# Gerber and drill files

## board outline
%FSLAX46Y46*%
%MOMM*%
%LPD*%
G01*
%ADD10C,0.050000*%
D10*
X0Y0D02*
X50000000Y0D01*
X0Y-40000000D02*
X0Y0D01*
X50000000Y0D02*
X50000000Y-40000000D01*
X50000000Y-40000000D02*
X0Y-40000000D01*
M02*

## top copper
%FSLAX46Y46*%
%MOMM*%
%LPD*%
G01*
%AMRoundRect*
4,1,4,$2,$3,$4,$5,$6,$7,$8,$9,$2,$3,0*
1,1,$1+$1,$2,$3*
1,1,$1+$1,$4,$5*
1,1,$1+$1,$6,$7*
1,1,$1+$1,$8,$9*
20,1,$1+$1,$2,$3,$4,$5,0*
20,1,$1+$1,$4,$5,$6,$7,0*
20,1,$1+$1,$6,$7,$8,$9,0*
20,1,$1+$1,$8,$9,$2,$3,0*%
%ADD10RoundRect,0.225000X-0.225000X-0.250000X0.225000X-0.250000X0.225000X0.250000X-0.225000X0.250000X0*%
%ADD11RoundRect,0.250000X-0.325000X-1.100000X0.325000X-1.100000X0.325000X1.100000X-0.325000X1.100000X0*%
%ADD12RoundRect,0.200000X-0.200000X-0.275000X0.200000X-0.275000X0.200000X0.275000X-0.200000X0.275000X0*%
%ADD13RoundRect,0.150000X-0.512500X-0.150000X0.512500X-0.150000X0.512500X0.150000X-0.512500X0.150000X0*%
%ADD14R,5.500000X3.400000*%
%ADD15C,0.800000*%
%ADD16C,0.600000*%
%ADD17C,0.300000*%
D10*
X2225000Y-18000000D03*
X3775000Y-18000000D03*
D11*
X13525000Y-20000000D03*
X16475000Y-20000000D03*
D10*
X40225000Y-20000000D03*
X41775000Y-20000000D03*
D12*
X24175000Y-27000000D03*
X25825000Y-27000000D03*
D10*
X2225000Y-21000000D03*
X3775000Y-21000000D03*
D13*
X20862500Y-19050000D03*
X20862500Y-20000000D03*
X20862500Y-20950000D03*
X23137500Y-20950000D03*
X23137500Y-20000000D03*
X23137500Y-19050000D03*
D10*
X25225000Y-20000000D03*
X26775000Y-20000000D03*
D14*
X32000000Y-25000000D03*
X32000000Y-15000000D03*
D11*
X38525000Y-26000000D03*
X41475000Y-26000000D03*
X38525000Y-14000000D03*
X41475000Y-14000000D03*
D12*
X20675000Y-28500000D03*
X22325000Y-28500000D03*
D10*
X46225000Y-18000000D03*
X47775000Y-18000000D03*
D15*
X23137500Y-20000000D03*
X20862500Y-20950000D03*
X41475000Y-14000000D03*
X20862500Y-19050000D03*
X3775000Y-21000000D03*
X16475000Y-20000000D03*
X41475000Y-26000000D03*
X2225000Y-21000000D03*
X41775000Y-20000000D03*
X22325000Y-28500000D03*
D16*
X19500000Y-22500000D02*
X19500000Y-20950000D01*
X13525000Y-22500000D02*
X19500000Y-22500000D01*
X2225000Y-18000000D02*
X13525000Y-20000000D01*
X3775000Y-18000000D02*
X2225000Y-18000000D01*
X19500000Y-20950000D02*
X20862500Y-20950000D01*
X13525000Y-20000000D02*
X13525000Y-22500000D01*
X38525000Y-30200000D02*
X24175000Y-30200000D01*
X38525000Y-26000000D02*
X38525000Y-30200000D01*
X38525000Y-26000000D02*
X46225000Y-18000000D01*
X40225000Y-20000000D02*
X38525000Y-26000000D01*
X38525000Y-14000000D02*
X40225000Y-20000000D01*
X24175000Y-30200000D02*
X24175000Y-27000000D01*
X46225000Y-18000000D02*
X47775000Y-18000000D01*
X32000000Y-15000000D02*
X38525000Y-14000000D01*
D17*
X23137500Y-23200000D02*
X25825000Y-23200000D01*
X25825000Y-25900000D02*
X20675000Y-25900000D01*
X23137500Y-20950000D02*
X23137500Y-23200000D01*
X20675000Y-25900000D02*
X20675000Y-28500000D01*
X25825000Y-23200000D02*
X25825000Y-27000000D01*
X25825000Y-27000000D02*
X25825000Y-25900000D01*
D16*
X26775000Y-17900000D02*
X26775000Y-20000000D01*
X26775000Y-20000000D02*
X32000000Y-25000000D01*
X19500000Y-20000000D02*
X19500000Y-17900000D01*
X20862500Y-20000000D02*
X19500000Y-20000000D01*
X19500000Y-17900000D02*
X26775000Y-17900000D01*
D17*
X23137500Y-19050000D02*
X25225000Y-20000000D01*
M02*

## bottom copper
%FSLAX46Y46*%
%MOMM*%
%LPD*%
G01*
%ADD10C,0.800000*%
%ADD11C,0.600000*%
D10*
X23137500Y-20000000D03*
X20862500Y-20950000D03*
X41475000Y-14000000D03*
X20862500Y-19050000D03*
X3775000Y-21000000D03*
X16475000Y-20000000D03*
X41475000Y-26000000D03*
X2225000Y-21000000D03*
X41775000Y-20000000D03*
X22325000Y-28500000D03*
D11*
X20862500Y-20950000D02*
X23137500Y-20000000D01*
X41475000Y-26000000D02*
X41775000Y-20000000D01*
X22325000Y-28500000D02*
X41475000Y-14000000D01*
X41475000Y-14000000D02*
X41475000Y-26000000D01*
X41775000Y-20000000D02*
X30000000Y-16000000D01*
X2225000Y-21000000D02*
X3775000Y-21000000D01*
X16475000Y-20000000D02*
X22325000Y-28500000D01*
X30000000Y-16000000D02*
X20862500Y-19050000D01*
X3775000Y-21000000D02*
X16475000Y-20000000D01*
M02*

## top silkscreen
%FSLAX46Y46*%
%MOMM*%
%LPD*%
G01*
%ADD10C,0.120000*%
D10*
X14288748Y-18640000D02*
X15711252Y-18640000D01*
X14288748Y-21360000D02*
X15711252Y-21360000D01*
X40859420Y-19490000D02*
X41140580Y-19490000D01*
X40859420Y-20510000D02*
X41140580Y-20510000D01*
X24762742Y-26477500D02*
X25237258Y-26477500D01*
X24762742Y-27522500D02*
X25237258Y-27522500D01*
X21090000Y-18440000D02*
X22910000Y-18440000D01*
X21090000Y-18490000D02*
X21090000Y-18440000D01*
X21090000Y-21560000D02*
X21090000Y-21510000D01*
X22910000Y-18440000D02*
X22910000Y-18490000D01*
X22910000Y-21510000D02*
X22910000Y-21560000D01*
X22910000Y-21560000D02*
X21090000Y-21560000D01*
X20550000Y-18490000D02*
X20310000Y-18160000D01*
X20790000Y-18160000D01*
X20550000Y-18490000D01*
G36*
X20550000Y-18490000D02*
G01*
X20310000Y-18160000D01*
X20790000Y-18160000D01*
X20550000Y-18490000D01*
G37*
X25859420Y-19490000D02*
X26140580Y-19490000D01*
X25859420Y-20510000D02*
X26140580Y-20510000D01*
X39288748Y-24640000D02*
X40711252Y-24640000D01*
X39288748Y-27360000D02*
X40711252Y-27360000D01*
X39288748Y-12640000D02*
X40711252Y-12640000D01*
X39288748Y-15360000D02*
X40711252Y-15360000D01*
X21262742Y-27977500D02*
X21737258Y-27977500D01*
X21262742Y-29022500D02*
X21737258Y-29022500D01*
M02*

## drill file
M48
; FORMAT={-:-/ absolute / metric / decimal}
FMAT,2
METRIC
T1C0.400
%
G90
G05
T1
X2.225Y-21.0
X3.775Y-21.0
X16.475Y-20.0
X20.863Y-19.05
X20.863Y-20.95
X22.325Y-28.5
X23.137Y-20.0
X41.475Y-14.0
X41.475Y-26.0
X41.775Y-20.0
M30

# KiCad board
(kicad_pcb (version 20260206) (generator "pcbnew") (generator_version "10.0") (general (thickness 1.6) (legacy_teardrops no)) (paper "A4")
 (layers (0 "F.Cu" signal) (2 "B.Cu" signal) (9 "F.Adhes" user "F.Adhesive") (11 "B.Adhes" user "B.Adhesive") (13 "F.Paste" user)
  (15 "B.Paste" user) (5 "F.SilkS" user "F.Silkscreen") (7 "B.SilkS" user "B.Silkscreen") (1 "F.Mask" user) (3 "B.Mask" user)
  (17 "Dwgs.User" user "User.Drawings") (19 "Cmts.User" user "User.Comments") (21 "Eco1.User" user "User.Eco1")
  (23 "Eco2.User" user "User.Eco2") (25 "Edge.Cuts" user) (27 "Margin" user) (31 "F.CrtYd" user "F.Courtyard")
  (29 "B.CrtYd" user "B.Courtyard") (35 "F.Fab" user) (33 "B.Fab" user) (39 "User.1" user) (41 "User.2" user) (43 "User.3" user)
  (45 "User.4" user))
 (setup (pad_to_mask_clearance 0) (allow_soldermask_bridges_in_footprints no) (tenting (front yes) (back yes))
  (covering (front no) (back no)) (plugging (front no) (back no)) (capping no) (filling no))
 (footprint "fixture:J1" (layer "F.Cu") (at 3 18)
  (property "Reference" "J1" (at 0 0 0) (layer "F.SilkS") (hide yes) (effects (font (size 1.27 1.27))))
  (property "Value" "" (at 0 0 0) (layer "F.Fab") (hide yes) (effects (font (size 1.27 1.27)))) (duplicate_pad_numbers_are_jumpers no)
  (pad "1" smd roundrect (at -0.775 0) (size 0.9 0.95) (layers "F.Cu" "F.Mask" "F.Paste") (roundrect_rratio 0.25) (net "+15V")
   (thermal_bridge_angle 45))
  (pad "2" smd roundrect (at 0.775 0) (size 0.9 0.95) (layers "F.Cu" "F.Mask" "F.Paste") (roundrect_rratio 0.25) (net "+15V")
   (thermal_bridge_angle 45)))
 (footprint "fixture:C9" (layer "F.Cu") (at 15 20)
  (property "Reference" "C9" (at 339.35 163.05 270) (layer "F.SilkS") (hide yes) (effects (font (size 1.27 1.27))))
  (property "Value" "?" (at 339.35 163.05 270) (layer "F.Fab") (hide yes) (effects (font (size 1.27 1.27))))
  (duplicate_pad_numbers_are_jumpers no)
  (fp_line (start -0.711252 -1.36) (end 0.711252 -1.36) (stroke (width 0.12) (type solid)) (layer "F.SilkS"))
  (fp_line (start -0.711252 1.36) (end 0.711252 1.36) (stroke (width 0.12) (type solid)) (layer "F.SilkS"))
  (pad "1" smd roundrect (at -1.475 0) (size 1.15 2.7) (layers "F.Cu" "F.Mask" "F.Paste") (roundrect_rratio 0.217391) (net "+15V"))
  (pad "2" smd roundrect (at 1.475 0) (size 1.15 2.7) (layers "F.Cu" "F.Mask" "F.Paste") (roundrect_rratio 0.217391) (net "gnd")))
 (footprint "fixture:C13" (layer "F.Cu") (at 41 20)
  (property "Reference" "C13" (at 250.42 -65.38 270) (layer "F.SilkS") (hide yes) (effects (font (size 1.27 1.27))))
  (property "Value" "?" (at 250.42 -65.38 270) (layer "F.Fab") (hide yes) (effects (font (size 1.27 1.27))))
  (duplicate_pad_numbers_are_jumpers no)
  (fp_line (start -0.14058 -0.51) (end 0.14058 -0.51) (stroke (width 0.12) (type solid)) (layer "F.SilkS"))
  (fp_line (start -0.14058 0.51) (end 0.14058 0.51) (stroke (width 0.12) (type solid)) (layer "F.SilkS"))
  (pad "1" smd roundrect (at -0.775 0) (size 0.9 0.95) (layers "F.Cu" "F.Mask" "F.Paste") (roundrect_rratio 0.25) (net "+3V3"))
  (pad "2" smd roundrect (at 0.775 0) (size 0.9 0.95) (layers "F.Cu" "F.Mask" "F.Paste") (roundrect_rratio 0.25) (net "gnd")))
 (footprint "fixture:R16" (layer "F.Cu") (at 25 27)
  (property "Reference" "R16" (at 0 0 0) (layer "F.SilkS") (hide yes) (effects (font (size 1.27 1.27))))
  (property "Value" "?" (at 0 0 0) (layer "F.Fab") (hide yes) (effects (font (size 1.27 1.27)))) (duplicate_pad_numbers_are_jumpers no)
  (fp_line (start -0.237258 -0.5225) (end 0.237258 -0.5225) (stroke (width 0.12) (type solid)) (layer "F.SilkS"))
  (fp_line (start -0.237258 0.5225) (end 0.237258 0.5225) (stroke (width 0.12) (type solid)) (layer "F.SilkS"))
  (pad "1" smd roundrect (at -0.825 0) (size 0.8 0.95) (layers "F.Cu" "F.Mask" "F.Paste") (roundrect_rratio 0.25) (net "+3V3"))
  (pad "2" smd roundrect (at 0.825 0) (size 0.8 0.95) (layers "F.Cu" "F.Mask" "F.Paste") (roundrect_rratio 0.25) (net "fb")))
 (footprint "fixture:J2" (layer "F.Cu") (at 3 21)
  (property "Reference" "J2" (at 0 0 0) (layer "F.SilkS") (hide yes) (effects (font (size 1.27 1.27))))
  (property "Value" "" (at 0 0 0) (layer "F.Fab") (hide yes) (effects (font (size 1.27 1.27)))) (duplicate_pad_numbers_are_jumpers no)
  (pad "1" smd roundrect (at -0.775 0) (size 0.9 0.95) (layers "F.Cu" "F.Mask" "F.Paste") (roundrect_rratio 0.25) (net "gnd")
   (thermal_bridge_angle 45))
  (pad "2" smd roundrect (at 0.775 0) (size 0.9 0.95) (layers "F.Cu" "F.Mask" "F.Paste") (roundrect_rratio 0.25) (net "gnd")
   (thermal_bridge_angle 45)))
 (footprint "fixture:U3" (layer "F.Cu") (at 22 20)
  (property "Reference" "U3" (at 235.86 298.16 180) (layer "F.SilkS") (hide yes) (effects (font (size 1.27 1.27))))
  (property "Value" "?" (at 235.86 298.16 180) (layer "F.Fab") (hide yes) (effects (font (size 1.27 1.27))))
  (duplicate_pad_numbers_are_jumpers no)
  (fp_line (start -0.91 -1.56) (end 0.91 -1.56) (stroke (width 0.12) (type solid)) (layer "F.SilkS"))
  (fp_line (start -0.91 -1.51) (end -0.91 -1.56) (stroke (width 0.12) (type solid)) (layer "F.SilkS"))
  (fp_line (start -0.91 1.56) (end -0.91 1.51) (stroke (width 0.12) (type solid)) (layer "F.SilkS"))
  (fp_line (start 0.91 -1.56) (end 0.91 -1.51) (stroke (width 0.12) (type solid)) (layer "F.SilkS"))
  (fp_line (start 0.91 1.51) (end 0.91 1.56) (stroke (width 0.12) (type solid)) (layer "F.SilkS"))
  (fp_line (start 0.91 1.56) (end -0.91 1.56) (stroke (width 0.12) (type solid)) (layer "F.SilkS"))
  (fp_poly (pts (xy -1.45 -1.51) (xy -1.69 -1.84) (xy -1.21 -1.84)) (stroke (width 0.12) (type solid)) (fill yes) (layer "F.SilkS"))
  (pad "1" smd roundrect (at -1.1375 -0.95) (size 1.325 0.6) (layers "F.Cu" "F.Mask" "F.Paste") (roundrect_rratio 0.25) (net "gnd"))
  (pad "2" smd roundrect (at -1.1375 0) (size 1.325 0.6) (layers "F.Cu" "F.Mask" "F.Paste") (roundrect_rratio 0.25) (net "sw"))
  (pad "3" smd roundrect (at -1.1375 0.95) (size 1.325 0.6) (layers "F.Cu" "F.Mask" "F.Paste") (roundrect_rratio 0.25) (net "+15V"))
  (pad "4" smd roundrect (at 1.1375 0.95) (size 1.325 0.6) (layers "F.Cu" "F.Mask" "F.Paste") (roundrect_rratio 0.25) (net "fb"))
  (pad "5" smd roundrect (at 1.1375 0) (size 1.325 0.6) (layers "F.Cu" "F.Mask" "F.Paste") (roundrect_rratio 0.25) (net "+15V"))
  (pad "6" smd roundrect (at 1.1375 -0.95) (size 1.325 0.6) (layers "F.Cu" "F.Mask" "F.Paste") (roundrect_rratio 0.25) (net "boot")))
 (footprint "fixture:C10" (layer "F.Cu") (at 26 20)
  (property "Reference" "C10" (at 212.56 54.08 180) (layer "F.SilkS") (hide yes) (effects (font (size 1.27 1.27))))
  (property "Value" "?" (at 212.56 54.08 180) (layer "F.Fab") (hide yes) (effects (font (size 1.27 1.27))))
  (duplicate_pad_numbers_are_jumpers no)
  (fp_line (start -0.14058 -0.51) (end 0.14058 -0.51) (stroke (width 0.12) (type solid)) (layer "F.SilkS"))
  (fp_line (start -0.14058 0.51) (end 0.14058 0.51) (stroke (width 0.12) (type solid)) (layer "F.SilkS"))
  (pad "1" smd roundrect (at -0.775 0) (size 0.9 0.95) (layers "F.Cu" "F.Mask" "F.Paste") (roundrect_rratio 0.25) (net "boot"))
  (pad "2" smd roundrect (at 0.775 0) (size 0.9 0.95) (layers "F.Cu" "F.Mask" "F.Paste") (roundrect_rratio 0.25) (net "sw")))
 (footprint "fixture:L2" (layer "F.Cu") (at 32 20 90)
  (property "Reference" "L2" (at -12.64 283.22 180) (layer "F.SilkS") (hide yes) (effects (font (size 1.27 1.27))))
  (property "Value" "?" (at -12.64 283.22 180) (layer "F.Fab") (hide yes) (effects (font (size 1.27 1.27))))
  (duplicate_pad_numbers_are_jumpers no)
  (pad "1" smd rect (at -5 0 90) (size 3.4 5.5) (layers "F.Cu" "F.Mask" "F.Paste") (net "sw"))
  (pad "2" smd rect (at 5 0 90) (size 3.4 5.5) (layers "F.Cu" "F.Mask" "F.Paste") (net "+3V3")))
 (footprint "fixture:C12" (layer "F.Cu") (at 40 26)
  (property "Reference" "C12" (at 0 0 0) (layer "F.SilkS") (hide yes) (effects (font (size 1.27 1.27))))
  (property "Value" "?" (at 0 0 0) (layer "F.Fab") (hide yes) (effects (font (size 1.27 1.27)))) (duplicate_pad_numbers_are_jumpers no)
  (fp_line (start -0.711252 -1.36) (end 0.711252 -1.36) (stroke (width 0.12) (type solid)) (layer "F.SilkS"))
  (fp_line (start -0.711252 1.36) (end 0.711252 1.36) (stroke (width 0.12) (type solid)) (layer "F.SilkS"))
  (pad "1" smd roundrect (at -1.475 0) (size 1.15 2.7) (layers "F.Cu" "F.Mask" "F.Paste") (roundrect_rratio 0.217391) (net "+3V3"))
  (pad "2" smd roundrect (at 1.475 0) (size 1.15 2.7) (layers "F.Cu" "F.Mask" "F.Paste") (roundrect_rratio 0.217391) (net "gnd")))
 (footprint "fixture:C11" (layer "F.Cu") (at 40 14)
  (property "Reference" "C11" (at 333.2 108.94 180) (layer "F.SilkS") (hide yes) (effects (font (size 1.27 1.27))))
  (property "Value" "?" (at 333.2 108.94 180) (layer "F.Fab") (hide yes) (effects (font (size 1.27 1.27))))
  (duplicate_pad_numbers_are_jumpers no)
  (fp_line (start -0.711252 -1.36) (end 0.711252 -1.36) (stroke (width 0.12) (type solid)) (layer "F.SilkS"))
  (fp_line (start -0.711252 1.36) (end 0.711252 1.36) (stroke (width 0.12) (type solid)) (layer "F.SilkS"))
  (pad "1" smd roundrect (at -1.475 0) (size 1.15 2.7) (layers "F.Cu" "F.Mask" "F.Paste") (roundrect_rratio 0.217391) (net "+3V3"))
  (pad "2" smd roundrect (at 1.475 0) (size 1.15 2.7) (layers "F.Cu" "F.Mask" "F.Paste") (roundrect_rratio 0.217391) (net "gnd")))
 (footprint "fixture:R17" (layer "F.Cu") (at 21.5 28.5)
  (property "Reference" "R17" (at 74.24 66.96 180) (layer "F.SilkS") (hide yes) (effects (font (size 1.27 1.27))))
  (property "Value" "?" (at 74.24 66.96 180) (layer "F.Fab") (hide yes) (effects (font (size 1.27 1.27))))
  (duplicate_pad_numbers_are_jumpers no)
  (fp_line (start -0.237258 -0.5225) (end 0.237258 -0.5225) (stroke (width 0.12) (type solid)) (layer "F.SilkS"))
  (fp_line (start -0.237258 0.5225) (end 0.237258 0.5225) (stroke (width 0.12) (type solid)) (layer "F.SilkS"))
  (pad "1" smd roundrect (at -0.825 0) (size 0.8 0.95) (layers "F.Cu" "F.Mask" "F.Paste") (roundrect_rratio 0.25) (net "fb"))
  (pad "2" smd roundrect (at 0.825 0) (size 0.8 0.95) (layers "F.Cu" "F.Mask" "F.Paste") (roundrect_rratio 0.25) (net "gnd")))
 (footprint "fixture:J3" (layer "F.Cu") (at 47 18)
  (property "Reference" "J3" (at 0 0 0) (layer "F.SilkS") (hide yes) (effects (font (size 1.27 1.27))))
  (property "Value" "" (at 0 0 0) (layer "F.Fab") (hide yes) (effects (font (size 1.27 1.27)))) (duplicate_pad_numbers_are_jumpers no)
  (pad "1" smd roundrect (at -0.775 0) (size 0.9 0.95) (layers "F.Cu" "F.Mask" "F.Paste") (roundrect_rratio 0.25) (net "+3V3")
   (thermal_bridge_angle 45))
  (pad "2" smd roundrect (at 0.775 0) (size 0.9 0.95) (layers "F.Cu" "F.Mask" "F.Paste") (roundrect_rratio 0.25) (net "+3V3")
   (thermal_bridge_angle 45)))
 (gr_line (start 0 0) (end 50 0) (stroke (width 0.05) (type default)) (layer "Edge.Cuts"))
 (gr_line (start 0 40) (end 0 0) (stroke (width 0.05) (type default)) (layer "Edge.Cuts"))
 (gr_line (start 50 0) (end 50 40) (stroke (width 0.05) (type default)) (layer "Edge.Cuts"))
 (gr_line (start 50 40) (end 0 40) (stroke (width 0.05) (type default)) (layer "Edge.Cuts"))
 (segment (start 19.5 22.5) (end 19.5 20.95) (width 0.6) (layer "F.Cu") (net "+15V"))
 (segment (start 13.525 22.5) (end 19.5 22.5) (width 0.6) (layer "F.Cu") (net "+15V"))
 (segment (start 2.225 18) (end 13.525 20) (width 0.6) (layer "F.Cu") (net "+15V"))
 (segment (start 3.775 18) (end 2.225 18) (width 0.6) (layer "F.Cu") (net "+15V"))
 (segment (start 19.5 20.95) (end 20.8625 20.95) (width 0.6) (layer "F.Cu") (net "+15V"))
 (segment (start 13.525 20) (end 13.525 22.5) (width 0.6) (layer "F.Cu") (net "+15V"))
 (via (at 23.1375 20) (size 0.8) (drill 0.4) (layers "F.Cu" "B.Cu") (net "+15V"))
 (via (at 20.8625 20.95) (size 0.8) (drill 0.4) (layers "F.Cu" "B.Cu") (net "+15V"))
 (segment (start 20.8625 20.95) (end 23.1375 20) (width 0.6) (layer "B.Cu") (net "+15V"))
 (via (at 41.475 14) (size 0.8) (drill 0.4) (layers "F.Cu" "B.Cu") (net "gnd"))
 (via (at 20.8625 19.05) (size 0.8) (drill 0.4) (layers "F.Cu" "B.Cu") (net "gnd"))
 (via (at 3.775 21) (size 0.8) (drill 0.4) (layers "F.Cu" "B.Cu") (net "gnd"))
 (via (at 16.475 20) (size 0.8) (drill 0.4) (layers "F.Cu" "B.Cu") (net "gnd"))
 (via (at 41.475 26) (size 0.8) (drill 0.4) (layers "F.Cu" "B.Cu") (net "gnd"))
 (via (at 2.225 21) (size 0.8) (drill 0.4) (layers "F.Cu" "B.Cu") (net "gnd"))
 (via (at 41.775 20) (size 0.8) (drill 0.4) (layers "F.Cu" "B.Cu") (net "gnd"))
 (via (at 22.325 28.5) (size 0.8) (drill 0.4) (layers "F.Cu" "B.Cu") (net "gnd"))
 (segment (start 41.475 26) (end 41.775 20) (width 0.6) (layer "B.Cu") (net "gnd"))
 (segment (start 22.325 28.5) (end 41.475 14) (width 0.6) (layer "B.Cu") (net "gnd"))
 (segment (start 41.475 14) (end 41.475 26) (width 0.6) (layer "B.Cu") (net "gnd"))
 (segment (start 41.775 20) (end 30 16) (width 0.6) (layer "B.Cu") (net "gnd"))
 (segment (start 2.225 21) (end 3.775 21) (width 0.6) (layer "B.Cu") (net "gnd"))
 (segment (start 16.475 20) (end 22.325 28.5) (width 0.6) (layer "B.Cu") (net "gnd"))
 (segment (start 30 16) (end 20.8625 19.05) (width 0.6) (layer "B.Cu") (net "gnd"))
 (segment (start 3.775 21) (end 16.475 20) (width 0.6) (layer "B.Cu") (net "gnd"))
 (segment (start 38.525 30.2) (end 24.175 30.2) (width 0.6) (layer "F.Cu") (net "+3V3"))
 (segment (start 38.525 26) (end 38.525 30.2) (width 0.6) (layer "F.Cu") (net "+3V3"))
 (segment (start 38.525 26) (end 46.225 18) (width 0.6) (layer "F.Cu") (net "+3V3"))
 (segment (start 40.225 20) (end 38.525 26) (width 0.6) (layer "F.Cu") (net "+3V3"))
 (segment (start 38.525 14) (end 40.225 20) (width 0.6) (layer "F.Cu") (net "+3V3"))
 (segment (start 24.175 30.2) (end 24.175 27) (width 0.6) (layer "F.Cu") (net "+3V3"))
 (segment (start 46.225 18) (end 47.775 18) (width 0.6) (layer "F.Cu") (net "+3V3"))
 (segment (start 32 15) (end 38.525 14) (width 0.6) (layer "F.Cu") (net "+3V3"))
 (segment (start 23.1375 23.2) (end 25.825 23.2) (width 0.3) (layer "F.Cu") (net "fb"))
 (segment (start 25.825 25.9) (end 20.675 25.9) (width 0.3) (layer "F.Cu") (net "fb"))
 (segment (start 23.1375 20.95) (end 23.1375 23.2) (width 0.3) (layer "F.Cu") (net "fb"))
 (segment (start 20.675 25.9) (end 20.675 28.5) (width 0.3) (layer "F.Cu") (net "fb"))
 (segment (start 25.825 23.2) (end 25.825 27) (width 0.3) (layer "F.Cu") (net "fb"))
 (segment (start 25.825 27) (end 25.825 25.9) (width 0.3) (layer "F.Cu") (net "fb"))
 (segment (start 26.775 17.9) (end 26.775 20) (width 0.6) (layer "F.Cu") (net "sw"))
 (segment (start 26.775 20) (end 32 25) (width 0.6) (layer "F.Cu") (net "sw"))
 (segment (start 19.5 20) (end 19.5 17.9) (width 0.6) (layer "F.Cu") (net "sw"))
 (segment (start 20.8625 20) (end 19.5 20) (width 0.6) (layer "F.Cu") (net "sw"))
 (segment (start 19.5 17.9) (end 26.775 17.9) (width 0.6) (layer "F.Cu") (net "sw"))
 (segment (start 23.1375 19.05) (end 25.225 20) (width 0.3) (layer "F.Cu") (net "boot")))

